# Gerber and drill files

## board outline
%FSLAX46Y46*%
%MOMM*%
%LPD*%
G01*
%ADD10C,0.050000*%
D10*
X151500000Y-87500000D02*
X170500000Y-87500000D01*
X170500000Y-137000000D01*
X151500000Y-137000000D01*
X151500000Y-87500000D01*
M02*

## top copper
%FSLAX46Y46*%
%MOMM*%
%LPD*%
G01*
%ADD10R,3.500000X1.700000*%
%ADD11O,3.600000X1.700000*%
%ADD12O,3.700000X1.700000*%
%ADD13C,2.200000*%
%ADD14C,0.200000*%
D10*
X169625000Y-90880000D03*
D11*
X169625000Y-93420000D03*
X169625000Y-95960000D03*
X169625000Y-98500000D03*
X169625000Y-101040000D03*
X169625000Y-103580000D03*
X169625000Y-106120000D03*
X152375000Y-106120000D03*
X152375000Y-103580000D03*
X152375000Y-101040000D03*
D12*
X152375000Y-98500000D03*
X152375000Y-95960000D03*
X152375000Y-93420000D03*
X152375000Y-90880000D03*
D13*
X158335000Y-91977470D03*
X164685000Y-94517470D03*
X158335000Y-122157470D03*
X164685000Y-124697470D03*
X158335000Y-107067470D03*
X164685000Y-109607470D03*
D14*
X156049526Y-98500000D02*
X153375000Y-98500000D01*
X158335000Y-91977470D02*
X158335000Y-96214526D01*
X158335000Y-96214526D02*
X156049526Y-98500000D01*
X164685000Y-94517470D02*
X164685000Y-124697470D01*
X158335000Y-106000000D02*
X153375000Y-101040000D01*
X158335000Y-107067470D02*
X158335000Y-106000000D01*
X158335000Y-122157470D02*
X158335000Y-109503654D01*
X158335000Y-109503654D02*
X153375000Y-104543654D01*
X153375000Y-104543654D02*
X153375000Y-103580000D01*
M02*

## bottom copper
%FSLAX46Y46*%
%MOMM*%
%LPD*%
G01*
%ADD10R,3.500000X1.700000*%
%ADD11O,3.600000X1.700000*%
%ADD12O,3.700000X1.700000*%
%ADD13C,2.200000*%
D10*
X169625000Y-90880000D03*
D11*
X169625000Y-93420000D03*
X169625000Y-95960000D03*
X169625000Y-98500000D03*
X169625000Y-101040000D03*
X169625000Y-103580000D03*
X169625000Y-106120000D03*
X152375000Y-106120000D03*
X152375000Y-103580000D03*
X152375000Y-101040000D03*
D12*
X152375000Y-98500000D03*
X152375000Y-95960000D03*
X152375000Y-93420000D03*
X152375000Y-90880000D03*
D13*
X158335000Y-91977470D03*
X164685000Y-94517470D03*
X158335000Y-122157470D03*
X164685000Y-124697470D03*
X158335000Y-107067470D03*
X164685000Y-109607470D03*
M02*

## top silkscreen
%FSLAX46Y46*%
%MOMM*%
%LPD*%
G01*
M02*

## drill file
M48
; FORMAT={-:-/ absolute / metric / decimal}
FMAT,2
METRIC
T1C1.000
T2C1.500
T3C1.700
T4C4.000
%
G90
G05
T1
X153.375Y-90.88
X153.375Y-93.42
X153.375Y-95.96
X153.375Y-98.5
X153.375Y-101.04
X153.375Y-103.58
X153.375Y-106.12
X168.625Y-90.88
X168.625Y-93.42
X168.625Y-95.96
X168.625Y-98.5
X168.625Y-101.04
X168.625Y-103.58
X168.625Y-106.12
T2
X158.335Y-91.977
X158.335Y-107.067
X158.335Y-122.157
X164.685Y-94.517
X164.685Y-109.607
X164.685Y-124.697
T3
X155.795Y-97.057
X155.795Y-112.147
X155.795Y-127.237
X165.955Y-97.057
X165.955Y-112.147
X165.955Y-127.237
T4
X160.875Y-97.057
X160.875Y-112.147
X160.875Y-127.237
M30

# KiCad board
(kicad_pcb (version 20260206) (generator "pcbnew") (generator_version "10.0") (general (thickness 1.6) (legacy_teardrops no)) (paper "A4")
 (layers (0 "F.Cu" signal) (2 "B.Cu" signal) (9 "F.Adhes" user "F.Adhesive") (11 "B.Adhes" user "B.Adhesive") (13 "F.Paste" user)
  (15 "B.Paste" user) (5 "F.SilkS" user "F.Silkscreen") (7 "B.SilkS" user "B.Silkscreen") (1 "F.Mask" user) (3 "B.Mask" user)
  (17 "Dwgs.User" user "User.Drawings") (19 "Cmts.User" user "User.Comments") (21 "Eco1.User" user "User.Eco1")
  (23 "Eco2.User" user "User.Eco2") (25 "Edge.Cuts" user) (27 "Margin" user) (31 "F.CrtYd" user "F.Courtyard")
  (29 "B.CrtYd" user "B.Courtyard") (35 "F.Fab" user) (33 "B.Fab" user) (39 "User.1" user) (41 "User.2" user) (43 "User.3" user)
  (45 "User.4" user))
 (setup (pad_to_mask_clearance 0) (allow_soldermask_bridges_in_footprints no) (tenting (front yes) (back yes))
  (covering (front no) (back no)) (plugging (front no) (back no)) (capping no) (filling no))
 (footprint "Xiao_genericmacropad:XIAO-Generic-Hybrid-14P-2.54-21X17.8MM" (layer "B.Cu") (at 161 98.5 180)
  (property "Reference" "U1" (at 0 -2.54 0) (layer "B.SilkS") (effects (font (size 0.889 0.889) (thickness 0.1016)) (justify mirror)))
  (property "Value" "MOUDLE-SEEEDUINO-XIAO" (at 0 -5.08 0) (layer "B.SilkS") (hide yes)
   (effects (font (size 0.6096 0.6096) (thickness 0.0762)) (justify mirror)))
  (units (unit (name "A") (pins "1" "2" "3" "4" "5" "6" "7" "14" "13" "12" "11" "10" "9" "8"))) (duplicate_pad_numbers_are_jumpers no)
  (pad "1" thru_hole rect (at -7.625 7.62 180) (size 3.5 1.7) (drill 1 (offset -1 0)) (layers "*.Cu" "*.Mask") (remove_unused_layers no)
   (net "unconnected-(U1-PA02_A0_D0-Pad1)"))
  (pad "2" thru_hole oval (at -7.625 5.08 180) (size 3.6 1.7) (drill 1 (offset -1 0)) (layers "*.Cu" "*.Mask") (remove_unused_layers no)
   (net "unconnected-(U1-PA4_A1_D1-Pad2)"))
  (pad "3" thru_hole oval (at -7.625 2.54 180) (size 3.6 1.7) (drill 1 (offset -1 0)) (layers "*.Cu" "*.Mask") (remove_unused_layers no)
   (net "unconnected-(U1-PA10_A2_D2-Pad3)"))
  (pad "4" thru_hole oval (at -7.625 0 180) (size 3.6 1.7) (drill 1 (offset -1 0)) (layers "*.Cu" "*.Mask") (remove_unused_layers no)
   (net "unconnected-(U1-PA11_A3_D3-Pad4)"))
  (pad "5" thru_hole oval (at -7.625 -2.54 180) (size 3.6 1.7) (drill 1 (offset -1 0)) (layers "*.Cu" "*.Mask") (remove_unused_layers no)
   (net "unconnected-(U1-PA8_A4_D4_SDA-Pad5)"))
  (pad "6" thru_hole oval (at -7.625 -5.08) (size 3.6 1.7) (drill 1 (offset 1 0)) (layers "*.Cu" "*.Mask") (remove_unused_layers no)
   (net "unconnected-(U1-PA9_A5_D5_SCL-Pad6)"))
  (pad "7" thru_hole oval (at -7.625 -7.62 180) (size 3.6 1.7) (drill 1 (offset -1 0)) (layers "*.Cu" "*.Mask") (remove_unused_layers no)
   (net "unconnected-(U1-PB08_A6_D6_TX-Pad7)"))
  (pad "8" thru_hole oval (at 7.625 -7.62 180) (size 3.6 1.7) (drill 1 (offset 1 0)) (layers "*.Cu" "*.Mask") (remove_unused_layers no)
   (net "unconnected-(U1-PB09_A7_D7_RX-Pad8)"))
  (pad "9" thru_hole oval (at 7.625 -5.08 180) (size 3.6 1.7) (drill 1 (offset 1 0)) (layers "*.Cu" "*.Mask") (remove_unused_layers no)
   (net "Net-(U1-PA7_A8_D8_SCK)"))
  (pad "10" thru_hole oval (at 7.625 -2.54 180) (size 3.6 1.7) (drill 1 (offset 1 0)) (layers "*.Cu" "*.Mask") (remove_unused_layers no)
   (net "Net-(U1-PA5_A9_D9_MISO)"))
  (pad "11" thru_hole oval (at 7.625 0 180) (size 3.7 1.7) (drill 1 (offset 1 0)) (layers "*.Cu" "*.Mask") (remove_unused_layers no)
   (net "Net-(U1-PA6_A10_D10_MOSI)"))
  (pad "12" thru_hole oval (at 7.625 2.54 180) (size 3.7 1.7) (drill 1 (offset 1 0)) (layers "*.Cu" "*.Mask") (remove_unused_layers no)
   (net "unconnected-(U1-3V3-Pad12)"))
  (pad "13" thru_hole oval (at 7.625 5.08 180) (size 3.7 1.7) (drill 1 (offset 1 0)) (layers "*.Cu" "*.Mask") (remove_unused_layers no)
   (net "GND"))
  (pad "14" thru_hole oval (at 7.625 7.62 180) (size 3.7 1.7) (drill 1 (offset 1 0)) (layers "*.Cu" "*.Mask") (remove_unused_layers no)
   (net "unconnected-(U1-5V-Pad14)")))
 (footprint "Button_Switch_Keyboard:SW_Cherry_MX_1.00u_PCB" (layer "B.Cu") (at 158.335 91.97747 180)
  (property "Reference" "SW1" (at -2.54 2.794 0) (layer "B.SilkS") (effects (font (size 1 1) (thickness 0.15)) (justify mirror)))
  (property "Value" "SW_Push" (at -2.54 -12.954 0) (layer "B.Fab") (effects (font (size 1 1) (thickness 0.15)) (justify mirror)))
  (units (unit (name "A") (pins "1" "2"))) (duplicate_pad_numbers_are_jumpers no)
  (pad "" np_thru_hole circle (at -7.62 -5.08 180) (size 1.7 1.7) (drill 1.7) (layers "*.Cu" "*.Mask"))
  (pad "" np_thru_hole circle (at -2.54 -5.08 180) (size 4 4) (drill 4) (layers "*.Cu" "*.Mask"))
  (pad "" np_thru_hole circle (at 2.54 -5.08 180) (size 1.7 1.7) (drill 1.7) (layers "*.Cu" "*.Mask"))
  (pad "1" thru_hole circle (at 0 0 180) (size 2.2 2.2) (drill 1.5) (layers "*.Cu" "*.Mask") (remove_unused_layers no)
   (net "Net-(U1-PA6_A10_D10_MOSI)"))
  (pad "2" thru_hole circle (at -6.35 -2.54 180) (size 2.2 2.2) (drill 1.5) (layers "*.Cu" "*.Mask") (remove_unused_layers no) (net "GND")))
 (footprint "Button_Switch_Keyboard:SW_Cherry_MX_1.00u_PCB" (layer "B.Cu") (at 158.335 122.15747 180)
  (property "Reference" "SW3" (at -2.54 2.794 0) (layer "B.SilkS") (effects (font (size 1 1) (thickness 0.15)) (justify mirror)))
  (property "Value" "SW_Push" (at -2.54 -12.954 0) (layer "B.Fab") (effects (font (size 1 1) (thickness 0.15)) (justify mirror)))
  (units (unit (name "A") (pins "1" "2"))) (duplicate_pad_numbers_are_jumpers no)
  (pad "" np_thru_hole circle (at -7.62 -5.08 180) (size 1.7 1.7) (drill 1.7) (layers "*.Cu" "*.Mask"))
  (pad "" np_thru_hole circle (at -2.54 -5.08 180) (size 4 4) (drill 4) (layers "*.Cu" "*.Mask"))
  (pad "" np_thru_hole circle (at 2.54 -5.08 180) (size 1.7 1.7) (drill 1.7) (layers "*.Cu" "*.Mask"))
  (pad "1" thru_hole circle (at 0 0 180) (size 2.2 2.2) (drill 1.5) (layers "*.Cu" "*.Mask") (remove_unused_layers no)
   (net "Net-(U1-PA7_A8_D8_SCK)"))
  (pad "2" thru_hole circle (at -6.35 -2.54 180) (size 2.2 2.2) (drill 1.5) (layers "*.Cu" "*.Mask") (remove_unused_layers no) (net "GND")))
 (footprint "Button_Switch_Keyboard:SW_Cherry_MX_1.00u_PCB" (layer "B.Cu") (at 158.335 107.06747 180)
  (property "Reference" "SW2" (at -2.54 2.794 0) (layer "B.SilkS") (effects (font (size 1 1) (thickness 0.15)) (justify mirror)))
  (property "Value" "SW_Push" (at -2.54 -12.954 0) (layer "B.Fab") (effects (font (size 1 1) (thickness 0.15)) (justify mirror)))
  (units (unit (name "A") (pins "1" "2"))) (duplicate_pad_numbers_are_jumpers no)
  (pad "" np_thru_hole circle (at -7.62 -5.08 180) (size 1.7 1.7) (drill 1.7) (layers "*.Cu" "*.Mask"))
  (pad "" np_thru_hole circle (at -2.54 -5.08 180) (size 4 4) (drill 4) (layers "*.Cu" "*.Mask"))
  (pad "" np_thru_hole circle (at 2.54 -5.08 180) (size 1.7 1.7) (drill 1.7) (layers "*.Cu" "*.Mask"))
  (pad "1" thru_hole circle (at 0 0 180) (size 2.2 2.2) (drill 1.5) (layers "*.Cu" "*.Mask") (remove_unused_layers no)
   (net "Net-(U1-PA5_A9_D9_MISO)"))
  (pad "2" thru_hole circle (at -6.35 -2.54 180) (size 2.2 2.2) (drill 1.5) (layers "*.Cu" "*.Mask") (remove_unused_layers no) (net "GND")))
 (gr_rect (start 151.5 87.5) (end 170.5 137) (stroke (width 0.05) (type default)) (fill no) (layer "Edge.Cuts"))
 (segment (start 156.049526 98.5) (end 153.375 98.5) (width 0.2) (layer "F.Cu") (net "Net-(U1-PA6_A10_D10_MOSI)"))
 (segment (start 158.335 91.97747) (end 158.335 96.214526) (width 0.2) (layer "F.Cu") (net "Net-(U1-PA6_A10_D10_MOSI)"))
 (segment (start 158.335 96.214526) (end 156.049526 98.5) (width 0.2) (layer "F.Cu") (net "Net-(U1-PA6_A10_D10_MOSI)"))
 (segment (start 164.685 94.51747) (end 164.685 124.69747) (width 0.2) (layer "F.Cu") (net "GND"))
 (segment (start 158.335 106) (end 153.375 101.04) (width 0.2) (layer "F.Cu") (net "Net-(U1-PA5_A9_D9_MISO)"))
 (segment (start 158.335 107.06747) (end 158.335 106) (width 0.2) (layer "F.Cu") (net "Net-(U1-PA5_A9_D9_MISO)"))
 (segment (start 158.335 122.15747) (end 158.335 109.503654) (width 0.2) (layer "F.Cu") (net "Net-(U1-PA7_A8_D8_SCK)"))
 (segment (start 158.335 109.503654) (end 153.375 104.543654) (width 0.2) (layer "F.Cu") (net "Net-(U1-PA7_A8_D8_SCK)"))
 (segment (start 153.375 104.543654) (end 153.375 103.58) (width 0.2) (layer "F.Cu") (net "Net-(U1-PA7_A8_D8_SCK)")))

